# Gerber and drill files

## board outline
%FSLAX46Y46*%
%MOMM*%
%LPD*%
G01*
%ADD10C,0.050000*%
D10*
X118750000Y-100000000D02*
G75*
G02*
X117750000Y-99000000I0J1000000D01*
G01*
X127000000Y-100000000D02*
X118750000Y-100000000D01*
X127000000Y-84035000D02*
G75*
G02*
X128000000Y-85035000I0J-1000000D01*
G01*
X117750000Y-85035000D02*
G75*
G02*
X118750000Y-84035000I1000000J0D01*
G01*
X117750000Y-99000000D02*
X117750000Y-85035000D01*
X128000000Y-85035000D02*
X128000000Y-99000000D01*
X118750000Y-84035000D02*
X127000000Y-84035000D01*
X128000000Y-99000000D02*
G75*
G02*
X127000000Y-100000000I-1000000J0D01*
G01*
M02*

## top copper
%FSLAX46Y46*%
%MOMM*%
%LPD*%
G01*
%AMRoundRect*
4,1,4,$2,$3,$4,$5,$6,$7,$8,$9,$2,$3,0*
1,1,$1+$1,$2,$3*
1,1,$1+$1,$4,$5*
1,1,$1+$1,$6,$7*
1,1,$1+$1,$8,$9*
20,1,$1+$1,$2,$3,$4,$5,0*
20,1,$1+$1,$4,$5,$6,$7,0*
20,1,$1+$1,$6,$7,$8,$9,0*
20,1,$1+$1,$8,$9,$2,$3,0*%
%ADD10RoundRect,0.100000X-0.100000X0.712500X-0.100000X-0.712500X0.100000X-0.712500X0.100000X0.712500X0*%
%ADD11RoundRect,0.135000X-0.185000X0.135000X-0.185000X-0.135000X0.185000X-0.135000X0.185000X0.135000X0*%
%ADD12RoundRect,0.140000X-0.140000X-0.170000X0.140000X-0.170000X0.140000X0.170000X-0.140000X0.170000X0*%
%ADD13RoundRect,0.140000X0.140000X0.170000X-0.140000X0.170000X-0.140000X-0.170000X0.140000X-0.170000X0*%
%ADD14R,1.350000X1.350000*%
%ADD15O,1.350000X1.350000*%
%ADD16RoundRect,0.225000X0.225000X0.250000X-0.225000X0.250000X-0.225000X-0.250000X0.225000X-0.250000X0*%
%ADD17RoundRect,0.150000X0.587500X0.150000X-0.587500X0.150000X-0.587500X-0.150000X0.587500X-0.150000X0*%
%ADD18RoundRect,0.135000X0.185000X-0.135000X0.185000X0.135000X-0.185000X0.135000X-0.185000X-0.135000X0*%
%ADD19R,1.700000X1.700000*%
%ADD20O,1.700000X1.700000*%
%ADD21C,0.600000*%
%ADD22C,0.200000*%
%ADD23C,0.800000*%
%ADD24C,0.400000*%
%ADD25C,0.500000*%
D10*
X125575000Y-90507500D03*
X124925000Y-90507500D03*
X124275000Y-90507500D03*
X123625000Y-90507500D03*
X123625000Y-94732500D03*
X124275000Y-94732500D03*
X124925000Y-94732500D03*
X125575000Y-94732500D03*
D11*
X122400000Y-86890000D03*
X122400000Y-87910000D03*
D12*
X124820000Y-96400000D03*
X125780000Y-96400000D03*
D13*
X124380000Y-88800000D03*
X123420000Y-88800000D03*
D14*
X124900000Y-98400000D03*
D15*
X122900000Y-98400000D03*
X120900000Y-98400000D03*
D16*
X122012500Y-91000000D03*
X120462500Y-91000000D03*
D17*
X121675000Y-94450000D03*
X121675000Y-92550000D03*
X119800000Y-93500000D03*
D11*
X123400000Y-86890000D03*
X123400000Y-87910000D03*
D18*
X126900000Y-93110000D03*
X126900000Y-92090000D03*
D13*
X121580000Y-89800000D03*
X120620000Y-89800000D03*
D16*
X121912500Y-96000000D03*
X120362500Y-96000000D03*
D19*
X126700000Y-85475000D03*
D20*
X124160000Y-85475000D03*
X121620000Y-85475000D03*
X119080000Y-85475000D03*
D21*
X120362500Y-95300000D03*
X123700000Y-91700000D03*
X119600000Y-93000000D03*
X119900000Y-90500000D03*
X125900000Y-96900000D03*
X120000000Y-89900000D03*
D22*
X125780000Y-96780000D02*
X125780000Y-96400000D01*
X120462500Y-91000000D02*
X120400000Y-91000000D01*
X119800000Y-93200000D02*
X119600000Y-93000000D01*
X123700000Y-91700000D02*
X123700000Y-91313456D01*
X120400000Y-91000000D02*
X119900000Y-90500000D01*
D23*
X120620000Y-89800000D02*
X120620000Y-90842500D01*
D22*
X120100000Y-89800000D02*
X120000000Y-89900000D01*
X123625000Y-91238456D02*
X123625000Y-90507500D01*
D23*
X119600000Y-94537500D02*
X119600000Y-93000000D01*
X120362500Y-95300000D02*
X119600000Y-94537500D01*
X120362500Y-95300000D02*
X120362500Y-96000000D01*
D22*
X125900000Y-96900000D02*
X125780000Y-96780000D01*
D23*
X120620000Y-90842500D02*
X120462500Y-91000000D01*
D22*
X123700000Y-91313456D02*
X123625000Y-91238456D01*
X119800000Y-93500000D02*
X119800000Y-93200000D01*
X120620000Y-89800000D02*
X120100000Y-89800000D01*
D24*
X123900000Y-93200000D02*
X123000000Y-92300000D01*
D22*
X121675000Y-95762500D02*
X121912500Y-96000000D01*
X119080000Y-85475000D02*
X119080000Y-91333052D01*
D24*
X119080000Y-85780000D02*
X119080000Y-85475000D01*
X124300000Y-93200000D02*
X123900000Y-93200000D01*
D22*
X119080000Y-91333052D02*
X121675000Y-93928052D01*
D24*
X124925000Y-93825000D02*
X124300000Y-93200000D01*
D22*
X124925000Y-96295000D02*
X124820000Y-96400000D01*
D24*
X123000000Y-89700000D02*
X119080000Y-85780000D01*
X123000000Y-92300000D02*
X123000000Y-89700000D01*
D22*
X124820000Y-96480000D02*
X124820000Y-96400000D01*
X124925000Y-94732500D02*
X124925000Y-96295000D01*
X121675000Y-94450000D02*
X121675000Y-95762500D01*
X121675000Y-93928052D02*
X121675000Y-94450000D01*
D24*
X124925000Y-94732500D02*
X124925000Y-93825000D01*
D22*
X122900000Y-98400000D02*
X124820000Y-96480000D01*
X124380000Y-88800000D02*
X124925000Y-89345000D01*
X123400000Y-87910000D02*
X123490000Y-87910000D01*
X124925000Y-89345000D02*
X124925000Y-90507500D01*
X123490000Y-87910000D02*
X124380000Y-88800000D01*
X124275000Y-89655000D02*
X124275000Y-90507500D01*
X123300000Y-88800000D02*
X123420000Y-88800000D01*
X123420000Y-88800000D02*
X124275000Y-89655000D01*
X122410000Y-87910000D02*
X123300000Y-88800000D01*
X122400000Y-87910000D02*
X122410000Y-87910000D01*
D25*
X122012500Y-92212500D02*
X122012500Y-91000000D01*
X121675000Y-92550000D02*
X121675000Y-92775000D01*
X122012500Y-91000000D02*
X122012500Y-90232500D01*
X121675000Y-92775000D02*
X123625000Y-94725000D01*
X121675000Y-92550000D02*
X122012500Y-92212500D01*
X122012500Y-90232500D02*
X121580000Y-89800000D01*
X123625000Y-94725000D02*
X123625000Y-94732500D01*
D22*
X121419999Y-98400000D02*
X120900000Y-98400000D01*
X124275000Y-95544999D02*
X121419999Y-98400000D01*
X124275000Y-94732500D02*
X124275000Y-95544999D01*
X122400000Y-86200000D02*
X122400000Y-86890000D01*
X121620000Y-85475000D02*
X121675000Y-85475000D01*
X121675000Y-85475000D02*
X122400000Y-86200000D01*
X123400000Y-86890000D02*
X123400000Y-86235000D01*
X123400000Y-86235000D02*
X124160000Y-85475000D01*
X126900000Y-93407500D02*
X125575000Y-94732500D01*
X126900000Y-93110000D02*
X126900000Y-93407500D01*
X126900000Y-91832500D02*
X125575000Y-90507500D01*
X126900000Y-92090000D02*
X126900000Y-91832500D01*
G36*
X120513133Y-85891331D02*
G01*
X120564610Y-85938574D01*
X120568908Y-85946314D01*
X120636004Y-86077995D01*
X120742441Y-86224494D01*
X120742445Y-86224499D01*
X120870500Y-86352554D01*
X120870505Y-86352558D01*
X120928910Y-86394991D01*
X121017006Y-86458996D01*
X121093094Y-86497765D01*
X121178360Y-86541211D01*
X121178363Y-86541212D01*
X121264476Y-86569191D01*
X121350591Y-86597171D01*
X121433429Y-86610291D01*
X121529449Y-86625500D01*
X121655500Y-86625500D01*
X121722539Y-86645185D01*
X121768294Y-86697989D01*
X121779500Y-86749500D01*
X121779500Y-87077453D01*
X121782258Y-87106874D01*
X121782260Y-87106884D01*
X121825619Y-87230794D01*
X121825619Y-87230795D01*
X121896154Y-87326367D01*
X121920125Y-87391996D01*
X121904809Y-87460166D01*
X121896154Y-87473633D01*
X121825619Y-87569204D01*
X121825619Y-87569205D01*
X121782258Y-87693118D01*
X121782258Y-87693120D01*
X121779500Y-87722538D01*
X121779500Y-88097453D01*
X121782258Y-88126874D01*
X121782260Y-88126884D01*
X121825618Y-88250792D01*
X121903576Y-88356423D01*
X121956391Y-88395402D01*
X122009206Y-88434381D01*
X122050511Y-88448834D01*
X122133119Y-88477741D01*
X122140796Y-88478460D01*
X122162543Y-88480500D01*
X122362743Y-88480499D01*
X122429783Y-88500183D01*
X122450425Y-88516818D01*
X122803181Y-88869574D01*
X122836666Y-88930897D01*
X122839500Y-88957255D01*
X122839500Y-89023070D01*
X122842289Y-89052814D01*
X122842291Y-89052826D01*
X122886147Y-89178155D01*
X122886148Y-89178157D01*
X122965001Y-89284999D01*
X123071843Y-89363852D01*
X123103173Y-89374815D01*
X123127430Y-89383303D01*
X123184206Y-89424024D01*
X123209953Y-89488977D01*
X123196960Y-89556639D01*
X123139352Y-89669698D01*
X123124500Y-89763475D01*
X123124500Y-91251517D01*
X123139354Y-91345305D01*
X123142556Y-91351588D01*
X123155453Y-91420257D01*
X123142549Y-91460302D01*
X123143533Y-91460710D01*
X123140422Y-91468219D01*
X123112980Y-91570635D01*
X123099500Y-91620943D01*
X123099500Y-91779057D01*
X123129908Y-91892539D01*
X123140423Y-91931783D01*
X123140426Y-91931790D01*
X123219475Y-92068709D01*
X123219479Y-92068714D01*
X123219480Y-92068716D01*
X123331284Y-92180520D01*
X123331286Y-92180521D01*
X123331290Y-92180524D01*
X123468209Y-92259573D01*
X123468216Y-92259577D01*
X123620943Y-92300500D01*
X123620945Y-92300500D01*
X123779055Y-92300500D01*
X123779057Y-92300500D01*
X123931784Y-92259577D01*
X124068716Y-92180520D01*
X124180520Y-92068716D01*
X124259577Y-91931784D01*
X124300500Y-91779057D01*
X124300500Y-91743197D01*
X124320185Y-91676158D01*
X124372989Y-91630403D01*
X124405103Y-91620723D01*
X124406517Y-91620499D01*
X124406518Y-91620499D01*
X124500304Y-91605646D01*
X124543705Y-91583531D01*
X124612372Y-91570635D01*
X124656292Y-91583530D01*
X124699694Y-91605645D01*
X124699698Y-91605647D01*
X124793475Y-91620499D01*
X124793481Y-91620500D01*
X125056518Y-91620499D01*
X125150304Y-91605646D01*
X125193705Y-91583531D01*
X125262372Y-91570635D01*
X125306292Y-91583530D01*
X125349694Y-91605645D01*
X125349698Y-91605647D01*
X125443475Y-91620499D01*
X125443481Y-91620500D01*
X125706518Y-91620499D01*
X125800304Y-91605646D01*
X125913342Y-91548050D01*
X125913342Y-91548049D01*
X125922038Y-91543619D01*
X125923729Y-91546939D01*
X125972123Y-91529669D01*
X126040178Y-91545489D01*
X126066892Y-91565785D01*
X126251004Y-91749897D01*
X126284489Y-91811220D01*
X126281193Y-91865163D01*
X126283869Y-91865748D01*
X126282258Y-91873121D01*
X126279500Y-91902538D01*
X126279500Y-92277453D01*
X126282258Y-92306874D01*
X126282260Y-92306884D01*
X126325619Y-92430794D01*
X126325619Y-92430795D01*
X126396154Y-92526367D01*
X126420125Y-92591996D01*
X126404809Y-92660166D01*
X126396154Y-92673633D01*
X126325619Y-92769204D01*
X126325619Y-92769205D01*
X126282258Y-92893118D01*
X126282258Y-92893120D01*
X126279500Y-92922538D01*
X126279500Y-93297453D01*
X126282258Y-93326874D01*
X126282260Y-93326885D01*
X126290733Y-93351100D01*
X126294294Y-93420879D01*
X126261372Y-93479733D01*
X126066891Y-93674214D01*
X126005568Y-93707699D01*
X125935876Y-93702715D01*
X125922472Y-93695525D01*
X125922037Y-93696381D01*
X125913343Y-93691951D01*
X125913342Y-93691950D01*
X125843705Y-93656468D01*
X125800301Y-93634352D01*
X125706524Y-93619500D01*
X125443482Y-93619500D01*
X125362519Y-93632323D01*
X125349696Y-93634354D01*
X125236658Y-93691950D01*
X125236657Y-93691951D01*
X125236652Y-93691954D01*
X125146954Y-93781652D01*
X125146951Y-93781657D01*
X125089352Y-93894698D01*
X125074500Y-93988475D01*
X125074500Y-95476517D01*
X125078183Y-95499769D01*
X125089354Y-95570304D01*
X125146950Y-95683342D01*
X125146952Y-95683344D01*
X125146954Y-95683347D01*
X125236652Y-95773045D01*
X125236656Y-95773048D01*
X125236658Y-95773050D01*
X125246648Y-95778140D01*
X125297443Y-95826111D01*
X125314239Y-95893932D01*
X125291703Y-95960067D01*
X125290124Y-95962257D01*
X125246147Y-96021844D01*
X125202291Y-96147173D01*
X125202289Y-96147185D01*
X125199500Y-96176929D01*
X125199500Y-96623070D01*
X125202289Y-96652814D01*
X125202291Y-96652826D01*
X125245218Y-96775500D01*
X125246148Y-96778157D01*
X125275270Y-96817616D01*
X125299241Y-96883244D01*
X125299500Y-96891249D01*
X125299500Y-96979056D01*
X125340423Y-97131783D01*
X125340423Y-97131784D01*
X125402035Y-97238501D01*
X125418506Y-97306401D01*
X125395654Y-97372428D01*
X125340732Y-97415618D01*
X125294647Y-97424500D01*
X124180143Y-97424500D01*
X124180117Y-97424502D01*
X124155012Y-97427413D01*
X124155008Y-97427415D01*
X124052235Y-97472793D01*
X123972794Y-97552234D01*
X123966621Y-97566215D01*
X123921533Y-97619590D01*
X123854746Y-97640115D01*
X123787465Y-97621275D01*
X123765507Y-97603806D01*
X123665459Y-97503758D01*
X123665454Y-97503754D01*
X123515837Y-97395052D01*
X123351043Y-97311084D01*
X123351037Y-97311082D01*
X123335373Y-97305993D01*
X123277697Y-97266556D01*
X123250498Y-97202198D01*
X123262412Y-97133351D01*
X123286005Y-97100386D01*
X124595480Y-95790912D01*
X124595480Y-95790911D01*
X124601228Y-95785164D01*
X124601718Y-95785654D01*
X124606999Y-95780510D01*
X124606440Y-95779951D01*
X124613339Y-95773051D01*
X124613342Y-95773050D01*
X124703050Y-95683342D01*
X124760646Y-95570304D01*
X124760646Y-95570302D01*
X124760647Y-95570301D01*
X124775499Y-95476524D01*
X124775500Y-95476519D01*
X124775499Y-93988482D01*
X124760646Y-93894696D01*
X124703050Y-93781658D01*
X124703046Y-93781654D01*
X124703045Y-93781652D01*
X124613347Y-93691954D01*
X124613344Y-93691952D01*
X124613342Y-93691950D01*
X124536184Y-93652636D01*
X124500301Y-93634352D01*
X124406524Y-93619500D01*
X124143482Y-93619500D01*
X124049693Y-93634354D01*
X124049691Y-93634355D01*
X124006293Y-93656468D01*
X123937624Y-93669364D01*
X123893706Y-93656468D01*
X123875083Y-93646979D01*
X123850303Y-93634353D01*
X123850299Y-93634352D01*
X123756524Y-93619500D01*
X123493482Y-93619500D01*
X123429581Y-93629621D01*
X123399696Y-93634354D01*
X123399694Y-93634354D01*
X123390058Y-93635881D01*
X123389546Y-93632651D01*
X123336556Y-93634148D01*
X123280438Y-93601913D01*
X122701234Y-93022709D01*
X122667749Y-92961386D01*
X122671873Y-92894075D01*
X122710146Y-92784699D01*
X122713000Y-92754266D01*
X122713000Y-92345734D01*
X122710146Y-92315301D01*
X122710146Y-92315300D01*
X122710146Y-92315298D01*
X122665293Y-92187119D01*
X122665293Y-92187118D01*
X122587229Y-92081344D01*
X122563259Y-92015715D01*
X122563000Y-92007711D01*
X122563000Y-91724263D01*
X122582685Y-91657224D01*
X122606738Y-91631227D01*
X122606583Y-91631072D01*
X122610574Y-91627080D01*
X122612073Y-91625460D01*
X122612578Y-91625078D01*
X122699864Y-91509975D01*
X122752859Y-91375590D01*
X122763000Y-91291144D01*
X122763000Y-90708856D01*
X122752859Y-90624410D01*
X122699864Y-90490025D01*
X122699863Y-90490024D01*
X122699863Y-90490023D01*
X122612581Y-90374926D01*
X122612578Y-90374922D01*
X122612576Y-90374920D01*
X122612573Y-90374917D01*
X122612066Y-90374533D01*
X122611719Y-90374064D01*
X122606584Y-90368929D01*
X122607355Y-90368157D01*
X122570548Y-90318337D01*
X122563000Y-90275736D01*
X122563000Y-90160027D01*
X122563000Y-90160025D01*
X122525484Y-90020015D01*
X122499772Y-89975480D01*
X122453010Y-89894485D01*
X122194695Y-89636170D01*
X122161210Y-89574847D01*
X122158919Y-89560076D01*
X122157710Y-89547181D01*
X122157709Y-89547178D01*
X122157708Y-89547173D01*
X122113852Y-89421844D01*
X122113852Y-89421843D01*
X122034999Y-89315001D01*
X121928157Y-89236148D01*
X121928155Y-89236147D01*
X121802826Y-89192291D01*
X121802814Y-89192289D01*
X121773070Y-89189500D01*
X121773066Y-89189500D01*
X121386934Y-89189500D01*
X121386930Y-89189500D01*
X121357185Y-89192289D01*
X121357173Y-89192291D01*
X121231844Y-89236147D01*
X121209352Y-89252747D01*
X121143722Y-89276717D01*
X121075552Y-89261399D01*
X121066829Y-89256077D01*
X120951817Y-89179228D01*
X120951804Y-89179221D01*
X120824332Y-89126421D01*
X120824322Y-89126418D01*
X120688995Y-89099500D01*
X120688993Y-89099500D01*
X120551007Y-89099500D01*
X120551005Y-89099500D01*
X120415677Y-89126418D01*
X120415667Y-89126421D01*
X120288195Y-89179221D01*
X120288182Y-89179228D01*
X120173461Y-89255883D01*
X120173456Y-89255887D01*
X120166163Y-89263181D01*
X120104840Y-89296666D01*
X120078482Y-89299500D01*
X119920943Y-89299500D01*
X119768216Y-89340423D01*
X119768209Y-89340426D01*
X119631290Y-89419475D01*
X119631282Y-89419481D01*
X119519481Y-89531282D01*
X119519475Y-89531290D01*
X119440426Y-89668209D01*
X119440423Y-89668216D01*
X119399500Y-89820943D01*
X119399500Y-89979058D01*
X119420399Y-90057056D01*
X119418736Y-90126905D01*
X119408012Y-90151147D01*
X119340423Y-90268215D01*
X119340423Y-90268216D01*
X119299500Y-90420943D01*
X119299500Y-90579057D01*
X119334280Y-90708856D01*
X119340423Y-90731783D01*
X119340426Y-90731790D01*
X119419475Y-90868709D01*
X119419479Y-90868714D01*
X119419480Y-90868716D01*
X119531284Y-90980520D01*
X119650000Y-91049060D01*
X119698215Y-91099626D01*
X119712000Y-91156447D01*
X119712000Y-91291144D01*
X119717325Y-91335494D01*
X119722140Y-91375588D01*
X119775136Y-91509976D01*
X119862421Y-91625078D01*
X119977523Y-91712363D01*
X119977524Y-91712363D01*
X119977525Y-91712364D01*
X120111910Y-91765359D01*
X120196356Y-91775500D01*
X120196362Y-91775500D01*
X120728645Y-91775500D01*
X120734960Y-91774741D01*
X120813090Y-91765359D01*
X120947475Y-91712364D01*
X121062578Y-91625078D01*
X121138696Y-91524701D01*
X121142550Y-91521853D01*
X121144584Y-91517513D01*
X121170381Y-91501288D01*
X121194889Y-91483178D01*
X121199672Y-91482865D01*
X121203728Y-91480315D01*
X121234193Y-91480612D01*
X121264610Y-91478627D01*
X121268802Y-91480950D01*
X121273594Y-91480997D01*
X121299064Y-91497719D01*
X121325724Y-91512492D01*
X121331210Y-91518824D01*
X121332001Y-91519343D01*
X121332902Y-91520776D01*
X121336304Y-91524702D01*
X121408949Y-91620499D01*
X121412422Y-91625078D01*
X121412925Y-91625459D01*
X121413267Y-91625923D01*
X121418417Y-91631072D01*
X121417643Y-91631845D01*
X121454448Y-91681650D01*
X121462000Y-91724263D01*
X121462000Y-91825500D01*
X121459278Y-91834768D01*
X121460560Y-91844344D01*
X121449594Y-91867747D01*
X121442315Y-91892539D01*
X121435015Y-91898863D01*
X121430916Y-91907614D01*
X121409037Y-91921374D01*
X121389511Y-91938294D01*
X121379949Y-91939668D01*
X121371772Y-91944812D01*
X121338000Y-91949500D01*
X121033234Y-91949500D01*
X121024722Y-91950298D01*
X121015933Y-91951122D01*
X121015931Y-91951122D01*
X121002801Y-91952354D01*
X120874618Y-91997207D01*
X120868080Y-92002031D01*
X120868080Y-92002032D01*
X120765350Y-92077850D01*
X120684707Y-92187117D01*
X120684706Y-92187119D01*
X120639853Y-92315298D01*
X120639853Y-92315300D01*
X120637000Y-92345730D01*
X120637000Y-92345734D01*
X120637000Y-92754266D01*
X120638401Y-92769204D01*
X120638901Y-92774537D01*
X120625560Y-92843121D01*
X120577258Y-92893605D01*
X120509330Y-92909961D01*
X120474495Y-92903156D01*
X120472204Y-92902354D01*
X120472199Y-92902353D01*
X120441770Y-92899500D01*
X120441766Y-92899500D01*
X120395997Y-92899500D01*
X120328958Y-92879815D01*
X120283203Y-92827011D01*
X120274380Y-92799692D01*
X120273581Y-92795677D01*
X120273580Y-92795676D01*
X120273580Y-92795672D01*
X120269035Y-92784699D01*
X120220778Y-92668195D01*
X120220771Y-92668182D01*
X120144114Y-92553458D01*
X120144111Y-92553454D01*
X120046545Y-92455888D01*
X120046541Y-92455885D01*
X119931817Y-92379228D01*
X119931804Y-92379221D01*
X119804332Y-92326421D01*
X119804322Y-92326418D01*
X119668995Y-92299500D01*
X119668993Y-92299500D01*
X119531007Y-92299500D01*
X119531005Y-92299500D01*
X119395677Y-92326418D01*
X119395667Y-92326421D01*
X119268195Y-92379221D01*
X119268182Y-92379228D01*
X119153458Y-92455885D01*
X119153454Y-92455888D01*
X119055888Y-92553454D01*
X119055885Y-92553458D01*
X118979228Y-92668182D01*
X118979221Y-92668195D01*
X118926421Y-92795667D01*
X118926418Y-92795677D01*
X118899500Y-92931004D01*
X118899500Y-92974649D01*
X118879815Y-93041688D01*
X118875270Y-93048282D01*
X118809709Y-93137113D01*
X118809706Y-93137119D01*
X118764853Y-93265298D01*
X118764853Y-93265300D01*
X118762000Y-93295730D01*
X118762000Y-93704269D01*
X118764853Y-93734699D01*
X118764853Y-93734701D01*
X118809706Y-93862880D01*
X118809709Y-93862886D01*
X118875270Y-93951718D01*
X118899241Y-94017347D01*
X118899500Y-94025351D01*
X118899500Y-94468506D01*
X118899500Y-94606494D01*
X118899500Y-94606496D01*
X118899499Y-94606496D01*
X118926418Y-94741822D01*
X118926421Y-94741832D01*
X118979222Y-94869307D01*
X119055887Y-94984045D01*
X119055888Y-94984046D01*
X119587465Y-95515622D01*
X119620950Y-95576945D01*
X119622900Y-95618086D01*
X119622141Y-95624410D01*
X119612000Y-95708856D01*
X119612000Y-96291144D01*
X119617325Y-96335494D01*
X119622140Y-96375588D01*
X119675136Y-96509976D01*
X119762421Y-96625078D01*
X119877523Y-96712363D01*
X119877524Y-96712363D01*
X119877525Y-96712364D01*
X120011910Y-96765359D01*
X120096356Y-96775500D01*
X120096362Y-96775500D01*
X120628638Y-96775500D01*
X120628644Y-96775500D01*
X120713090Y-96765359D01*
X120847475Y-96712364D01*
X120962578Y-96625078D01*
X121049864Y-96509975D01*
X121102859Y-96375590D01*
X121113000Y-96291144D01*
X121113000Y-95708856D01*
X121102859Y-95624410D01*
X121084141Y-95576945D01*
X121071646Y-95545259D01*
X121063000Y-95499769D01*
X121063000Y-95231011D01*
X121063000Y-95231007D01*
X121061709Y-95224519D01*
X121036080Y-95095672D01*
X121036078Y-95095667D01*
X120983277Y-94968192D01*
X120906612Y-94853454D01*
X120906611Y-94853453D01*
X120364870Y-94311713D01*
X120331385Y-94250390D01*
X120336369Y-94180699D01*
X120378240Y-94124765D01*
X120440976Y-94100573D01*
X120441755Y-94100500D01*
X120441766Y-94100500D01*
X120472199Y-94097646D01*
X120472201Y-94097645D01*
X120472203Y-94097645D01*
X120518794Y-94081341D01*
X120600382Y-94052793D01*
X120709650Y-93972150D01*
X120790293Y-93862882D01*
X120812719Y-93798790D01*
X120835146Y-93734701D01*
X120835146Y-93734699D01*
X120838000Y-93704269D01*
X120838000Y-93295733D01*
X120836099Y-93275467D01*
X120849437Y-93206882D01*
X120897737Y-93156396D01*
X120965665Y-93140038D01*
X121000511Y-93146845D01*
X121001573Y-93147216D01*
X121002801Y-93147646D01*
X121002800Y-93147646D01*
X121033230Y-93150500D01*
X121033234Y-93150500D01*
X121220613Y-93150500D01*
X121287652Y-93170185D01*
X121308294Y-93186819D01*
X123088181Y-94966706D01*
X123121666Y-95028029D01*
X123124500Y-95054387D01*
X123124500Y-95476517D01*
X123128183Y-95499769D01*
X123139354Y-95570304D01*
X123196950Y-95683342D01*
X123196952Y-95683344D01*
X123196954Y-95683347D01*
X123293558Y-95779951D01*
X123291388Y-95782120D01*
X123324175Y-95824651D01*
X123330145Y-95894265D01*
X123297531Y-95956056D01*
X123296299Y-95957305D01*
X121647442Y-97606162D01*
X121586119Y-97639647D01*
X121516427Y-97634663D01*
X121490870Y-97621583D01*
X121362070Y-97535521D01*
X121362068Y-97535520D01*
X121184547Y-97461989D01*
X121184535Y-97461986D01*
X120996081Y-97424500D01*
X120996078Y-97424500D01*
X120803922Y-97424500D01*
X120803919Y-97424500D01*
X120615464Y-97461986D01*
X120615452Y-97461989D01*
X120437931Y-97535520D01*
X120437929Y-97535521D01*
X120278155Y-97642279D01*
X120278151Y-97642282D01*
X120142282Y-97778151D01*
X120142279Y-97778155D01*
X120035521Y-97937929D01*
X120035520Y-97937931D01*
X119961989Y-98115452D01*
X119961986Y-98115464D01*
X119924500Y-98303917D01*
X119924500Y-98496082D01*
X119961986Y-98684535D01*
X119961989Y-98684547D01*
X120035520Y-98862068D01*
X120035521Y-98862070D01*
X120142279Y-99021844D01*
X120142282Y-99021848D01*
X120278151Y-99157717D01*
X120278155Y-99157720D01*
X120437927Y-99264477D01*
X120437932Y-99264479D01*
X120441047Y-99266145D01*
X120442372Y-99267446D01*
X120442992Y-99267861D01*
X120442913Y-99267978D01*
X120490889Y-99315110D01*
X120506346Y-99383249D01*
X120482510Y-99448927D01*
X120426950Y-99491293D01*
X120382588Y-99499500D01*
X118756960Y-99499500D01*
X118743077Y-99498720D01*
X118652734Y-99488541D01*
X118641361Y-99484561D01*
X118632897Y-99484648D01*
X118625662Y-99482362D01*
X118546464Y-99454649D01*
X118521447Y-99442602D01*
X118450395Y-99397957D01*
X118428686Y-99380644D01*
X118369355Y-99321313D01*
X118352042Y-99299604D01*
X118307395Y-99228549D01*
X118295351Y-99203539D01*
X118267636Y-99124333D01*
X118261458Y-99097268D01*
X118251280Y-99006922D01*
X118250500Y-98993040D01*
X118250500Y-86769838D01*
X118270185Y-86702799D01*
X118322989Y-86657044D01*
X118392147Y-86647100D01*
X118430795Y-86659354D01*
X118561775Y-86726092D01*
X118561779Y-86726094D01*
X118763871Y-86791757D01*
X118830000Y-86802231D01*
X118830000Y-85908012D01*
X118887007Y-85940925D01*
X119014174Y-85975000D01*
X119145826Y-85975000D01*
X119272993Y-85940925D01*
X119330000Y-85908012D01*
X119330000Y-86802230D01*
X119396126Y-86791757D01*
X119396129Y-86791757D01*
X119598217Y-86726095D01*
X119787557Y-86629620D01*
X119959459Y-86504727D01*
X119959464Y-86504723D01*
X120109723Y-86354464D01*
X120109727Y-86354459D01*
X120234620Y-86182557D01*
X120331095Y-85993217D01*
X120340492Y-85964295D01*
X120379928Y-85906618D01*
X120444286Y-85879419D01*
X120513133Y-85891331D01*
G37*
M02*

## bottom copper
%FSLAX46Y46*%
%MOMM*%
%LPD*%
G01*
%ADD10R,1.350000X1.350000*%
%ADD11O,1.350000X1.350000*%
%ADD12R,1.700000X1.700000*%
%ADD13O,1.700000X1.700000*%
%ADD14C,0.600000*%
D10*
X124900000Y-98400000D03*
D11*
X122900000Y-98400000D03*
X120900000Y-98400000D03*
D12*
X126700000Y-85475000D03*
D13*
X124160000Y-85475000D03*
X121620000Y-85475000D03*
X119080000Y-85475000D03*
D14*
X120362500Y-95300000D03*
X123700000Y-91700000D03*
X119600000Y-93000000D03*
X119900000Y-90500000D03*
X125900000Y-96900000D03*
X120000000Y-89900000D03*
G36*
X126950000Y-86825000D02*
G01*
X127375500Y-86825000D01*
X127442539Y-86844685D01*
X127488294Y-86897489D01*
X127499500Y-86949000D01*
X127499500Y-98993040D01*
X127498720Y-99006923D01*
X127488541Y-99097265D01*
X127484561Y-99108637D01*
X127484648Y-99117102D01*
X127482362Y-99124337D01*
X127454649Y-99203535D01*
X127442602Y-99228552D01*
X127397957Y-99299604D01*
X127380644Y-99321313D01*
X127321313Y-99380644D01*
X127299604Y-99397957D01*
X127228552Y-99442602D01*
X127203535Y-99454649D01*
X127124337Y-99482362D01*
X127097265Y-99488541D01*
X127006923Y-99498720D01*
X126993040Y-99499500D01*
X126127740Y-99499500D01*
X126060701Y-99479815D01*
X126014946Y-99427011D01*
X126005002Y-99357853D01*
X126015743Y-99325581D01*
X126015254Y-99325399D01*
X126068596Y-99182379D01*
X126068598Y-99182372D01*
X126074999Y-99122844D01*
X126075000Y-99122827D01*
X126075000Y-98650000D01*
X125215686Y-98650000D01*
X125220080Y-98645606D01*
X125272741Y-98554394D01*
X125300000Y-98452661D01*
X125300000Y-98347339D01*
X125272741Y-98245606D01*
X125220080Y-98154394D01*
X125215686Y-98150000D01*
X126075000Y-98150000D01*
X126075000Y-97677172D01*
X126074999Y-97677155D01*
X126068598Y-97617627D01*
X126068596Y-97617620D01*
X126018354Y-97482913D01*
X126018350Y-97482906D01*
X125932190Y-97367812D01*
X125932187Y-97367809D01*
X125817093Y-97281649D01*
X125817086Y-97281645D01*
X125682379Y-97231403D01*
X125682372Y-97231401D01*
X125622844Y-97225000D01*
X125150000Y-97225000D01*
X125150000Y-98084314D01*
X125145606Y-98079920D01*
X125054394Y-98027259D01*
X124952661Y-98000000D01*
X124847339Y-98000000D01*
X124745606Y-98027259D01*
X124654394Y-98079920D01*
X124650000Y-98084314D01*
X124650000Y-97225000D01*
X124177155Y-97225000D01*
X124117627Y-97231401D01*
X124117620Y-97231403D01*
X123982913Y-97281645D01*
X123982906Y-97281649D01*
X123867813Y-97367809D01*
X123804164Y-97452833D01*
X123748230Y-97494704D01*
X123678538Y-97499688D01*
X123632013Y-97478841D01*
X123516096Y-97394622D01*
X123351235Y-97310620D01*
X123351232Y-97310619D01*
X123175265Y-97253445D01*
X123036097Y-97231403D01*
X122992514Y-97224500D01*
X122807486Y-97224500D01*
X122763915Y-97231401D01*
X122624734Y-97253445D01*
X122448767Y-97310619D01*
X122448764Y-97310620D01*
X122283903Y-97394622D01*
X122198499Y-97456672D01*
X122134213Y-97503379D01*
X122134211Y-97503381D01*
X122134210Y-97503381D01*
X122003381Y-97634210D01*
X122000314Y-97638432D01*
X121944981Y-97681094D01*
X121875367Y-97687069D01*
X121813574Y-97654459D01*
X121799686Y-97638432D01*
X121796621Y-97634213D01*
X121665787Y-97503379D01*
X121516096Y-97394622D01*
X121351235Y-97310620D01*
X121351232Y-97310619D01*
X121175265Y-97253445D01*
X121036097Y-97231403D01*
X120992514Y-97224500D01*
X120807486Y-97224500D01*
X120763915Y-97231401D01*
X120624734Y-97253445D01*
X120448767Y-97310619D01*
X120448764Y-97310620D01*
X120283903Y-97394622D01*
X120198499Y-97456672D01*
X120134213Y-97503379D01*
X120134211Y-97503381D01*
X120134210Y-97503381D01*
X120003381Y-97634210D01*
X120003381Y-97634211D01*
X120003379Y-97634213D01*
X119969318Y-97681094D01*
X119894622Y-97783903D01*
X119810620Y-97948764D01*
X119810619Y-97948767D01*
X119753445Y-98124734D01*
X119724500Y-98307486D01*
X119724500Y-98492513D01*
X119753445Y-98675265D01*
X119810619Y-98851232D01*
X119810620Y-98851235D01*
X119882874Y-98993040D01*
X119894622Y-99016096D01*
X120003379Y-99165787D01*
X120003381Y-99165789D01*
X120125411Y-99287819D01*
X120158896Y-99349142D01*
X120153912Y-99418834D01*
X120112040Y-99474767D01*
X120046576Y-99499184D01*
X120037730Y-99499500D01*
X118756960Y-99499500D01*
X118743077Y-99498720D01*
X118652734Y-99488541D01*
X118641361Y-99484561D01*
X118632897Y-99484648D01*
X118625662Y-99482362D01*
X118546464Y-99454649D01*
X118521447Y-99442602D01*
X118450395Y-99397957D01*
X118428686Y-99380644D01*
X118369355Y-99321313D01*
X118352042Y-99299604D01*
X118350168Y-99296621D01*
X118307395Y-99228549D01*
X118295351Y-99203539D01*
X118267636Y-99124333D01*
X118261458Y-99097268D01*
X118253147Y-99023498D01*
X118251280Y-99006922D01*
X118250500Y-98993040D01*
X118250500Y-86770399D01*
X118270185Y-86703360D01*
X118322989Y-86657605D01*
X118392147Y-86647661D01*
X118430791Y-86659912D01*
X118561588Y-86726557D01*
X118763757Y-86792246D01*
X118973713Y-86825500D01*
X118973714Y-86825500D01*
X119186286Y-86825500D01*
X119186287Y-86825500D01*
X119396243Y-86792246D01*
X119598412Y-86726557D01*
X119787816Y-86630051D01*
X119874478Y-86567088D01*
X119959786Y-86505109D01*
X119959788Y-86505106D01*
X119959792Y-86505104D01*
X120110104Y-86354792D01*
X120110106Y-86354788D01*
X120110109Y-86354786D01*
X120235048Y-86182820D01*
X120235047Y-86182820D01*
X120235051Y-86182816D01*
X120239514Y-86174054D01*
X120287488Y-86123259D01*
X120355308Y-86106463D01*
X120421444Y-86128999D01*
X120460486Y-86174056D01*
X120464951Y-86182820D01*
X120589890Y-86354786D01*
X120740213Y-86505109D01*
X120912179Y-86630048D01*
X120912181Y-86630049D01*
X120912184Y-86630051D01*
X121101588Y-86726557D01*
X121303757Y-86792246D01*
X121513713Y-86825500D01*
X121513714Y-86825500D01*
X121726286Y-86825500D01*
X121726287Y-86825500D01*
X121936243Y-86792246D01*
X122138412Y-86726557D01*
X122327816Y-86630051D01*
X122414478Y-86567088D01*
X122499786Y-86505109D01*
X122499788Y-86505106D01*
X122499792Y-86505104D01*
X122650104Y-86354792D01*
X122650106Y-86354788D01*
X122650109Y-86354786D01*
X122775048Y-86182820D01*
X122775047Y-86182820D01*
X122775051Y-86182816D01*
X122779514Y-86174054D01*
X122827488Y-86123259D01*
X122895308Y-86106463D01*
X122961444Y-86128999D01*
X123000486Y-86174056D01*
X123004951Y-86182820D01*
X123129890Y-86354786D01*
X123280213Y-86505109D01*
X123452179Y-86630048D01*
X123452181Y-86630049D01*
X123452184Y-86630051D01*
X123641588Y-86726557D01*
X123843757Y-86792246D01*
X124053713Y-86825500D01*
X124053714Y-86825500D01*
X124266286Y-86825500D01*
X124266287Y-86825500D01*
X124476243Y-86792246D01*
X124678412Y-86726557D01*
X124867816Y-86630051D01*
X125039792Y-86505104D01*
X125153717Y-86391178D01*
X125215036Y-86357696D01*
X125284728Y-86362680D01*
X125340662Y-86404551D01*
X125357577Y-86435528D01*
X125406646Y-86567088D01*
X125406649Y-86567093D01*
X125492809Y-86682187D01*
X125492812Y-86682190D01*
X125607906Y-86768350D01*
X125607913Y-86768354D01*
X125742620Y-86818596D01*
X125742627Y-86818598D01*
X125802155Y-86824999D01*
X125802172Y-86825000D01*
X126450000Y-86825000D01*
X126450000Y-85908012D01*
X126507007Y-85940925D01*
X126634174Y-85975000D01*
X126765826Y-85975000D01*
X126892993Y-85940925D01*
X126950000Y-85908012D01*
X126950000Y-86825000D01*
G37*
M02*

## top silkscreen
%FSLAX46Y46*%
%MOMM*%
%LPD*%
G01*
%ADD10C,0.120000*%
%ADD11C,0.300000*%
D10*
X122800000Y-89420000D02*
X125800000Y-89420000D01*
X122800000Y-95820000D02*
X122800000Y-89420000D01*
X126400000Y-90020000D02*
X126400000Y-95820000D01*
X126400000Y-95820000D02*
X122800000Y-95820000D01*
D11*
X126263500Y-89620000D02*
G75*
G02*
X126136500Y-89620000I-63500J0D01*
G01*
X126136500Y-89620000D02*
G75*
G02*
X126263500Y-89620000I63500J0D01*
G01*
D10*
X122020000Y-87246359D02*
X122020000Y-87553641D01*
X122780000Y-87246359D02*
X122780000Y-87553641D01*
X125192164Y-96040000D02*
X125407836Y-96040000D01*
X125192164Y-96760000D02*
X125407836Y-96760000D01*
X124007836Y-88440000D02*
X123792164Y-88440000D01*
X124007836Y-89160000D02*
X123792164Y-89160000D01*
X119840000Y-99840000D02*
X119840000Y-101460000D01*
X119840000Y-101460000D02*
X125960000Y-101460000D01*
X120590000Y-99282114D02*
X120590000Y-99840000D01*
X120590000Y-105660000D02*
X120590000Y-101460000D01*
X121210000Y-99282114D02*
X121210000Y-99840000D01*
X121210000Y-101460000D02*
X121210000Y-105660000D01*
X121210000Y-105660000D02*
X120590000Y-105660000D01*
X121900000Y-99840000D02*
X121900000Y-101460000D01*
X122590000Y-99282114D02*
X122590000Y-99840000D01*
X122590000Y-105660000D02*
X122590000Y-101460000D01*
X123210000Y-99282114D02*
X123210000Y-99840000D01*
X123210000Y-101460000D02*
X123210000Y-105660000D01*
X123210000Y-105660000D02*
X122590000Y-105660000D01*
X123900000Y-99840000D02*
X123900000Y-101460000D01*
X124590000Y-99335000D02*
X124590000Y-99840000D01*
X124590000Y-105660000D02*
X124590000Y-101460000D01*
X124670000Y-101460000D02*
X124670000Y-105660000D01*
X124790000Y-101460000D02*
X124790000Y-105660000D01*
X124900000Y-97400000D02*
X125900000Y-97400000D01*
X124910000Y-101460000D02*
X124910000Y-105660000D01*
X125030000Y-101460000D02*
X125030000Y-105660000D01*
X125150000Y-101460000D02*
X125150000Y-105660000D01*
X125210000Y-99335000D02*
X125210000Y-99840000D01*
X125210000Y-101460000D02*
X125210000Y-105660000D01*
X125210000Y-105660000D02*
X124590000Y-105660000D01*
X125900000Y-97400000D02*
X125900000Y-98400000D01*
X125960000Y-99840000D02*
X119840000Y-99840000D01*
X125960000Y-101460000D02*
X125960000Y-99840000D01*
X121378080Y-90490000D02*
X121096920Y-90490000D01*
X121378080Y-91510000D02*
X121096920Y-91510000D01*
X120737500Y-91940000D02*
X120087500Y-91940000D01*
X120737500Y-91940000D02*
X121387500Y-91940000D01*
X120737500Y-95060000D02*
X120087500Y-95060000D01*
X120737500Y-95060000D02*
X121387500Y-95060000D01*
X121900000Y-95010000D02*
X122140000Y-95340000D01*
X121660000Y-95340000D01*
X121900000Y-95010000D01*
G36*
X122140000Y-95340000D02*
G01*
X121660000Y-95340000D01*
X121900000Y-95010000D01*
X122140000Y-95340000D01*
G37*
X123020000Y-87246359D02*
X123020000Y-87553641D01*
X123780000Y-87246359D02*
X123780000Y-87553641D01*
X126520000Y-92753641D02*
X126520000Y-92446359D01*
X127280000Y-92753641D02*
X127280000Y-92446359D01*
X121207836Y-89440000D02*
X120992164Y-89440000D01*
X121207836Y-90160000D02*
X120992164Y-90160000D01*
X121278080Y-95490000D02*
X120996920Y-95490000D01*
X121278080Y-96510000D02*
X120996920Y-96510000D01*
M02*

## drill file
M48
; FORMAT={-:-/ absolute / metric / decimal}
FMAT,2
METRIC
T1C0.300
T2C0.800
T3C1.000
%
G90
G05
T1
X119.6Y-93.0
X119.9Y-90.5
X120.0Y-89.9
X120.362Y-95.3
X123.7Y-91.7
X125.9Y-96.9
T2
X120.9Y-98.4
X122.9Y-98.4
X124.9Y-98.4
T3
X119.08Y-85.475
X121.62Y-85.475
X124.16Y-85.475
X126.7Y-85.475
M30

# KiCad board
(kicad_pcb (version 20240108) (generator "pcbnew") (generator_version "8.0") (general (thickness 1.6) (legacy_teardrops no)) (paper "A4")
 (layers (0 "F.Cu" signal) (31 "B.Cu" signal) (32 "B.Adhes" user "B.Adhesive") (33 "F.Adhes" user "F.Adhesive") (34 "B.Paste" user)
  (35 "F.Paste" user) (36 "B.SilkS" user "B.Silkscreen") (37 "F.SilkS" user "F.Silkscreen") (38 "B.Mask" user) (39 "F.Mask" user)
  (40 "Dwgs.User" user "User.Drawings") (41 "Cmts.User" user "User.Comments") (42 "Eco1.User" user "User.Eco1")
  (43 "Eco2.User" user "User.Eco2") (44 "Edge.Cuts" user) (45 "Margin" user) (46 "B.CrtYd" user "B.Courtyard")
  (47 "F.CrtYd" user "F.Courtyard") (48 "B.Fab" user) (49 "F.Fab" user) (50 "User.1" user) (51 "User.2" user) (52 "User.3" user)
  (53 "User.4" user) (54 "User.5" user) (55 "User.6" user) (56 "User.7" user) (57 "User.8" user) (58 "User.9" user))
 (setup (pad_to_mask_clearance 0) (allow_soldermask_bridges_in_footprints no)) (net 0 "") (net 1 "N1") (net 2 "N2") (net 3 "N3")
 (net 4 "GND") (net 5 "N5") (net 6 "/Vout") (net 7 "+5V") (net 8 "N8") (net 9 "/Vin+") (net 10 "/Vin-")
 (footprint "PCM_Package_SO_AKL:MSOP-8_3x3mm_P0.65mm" (layer "F.Cu") (at 124.6 92.62 -90)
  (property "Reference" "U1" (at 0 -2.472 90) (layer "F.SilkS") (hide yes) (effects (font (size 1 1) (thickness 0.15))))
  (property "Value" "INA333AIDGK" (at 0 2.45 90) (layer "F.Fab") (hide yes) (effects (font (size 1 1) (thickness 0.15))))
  (fp_line (start -3.2 1.8) (end -3.2 -1.2) (stroke (width 0.12) (type solid)) (layer "F.SilkS"))
  (fp_line (start 3.2 1.8) (end -3.2 1.8) (stroke (width 0.12) (type solid)) (layer "F.SilkS"))
  (fp_line (start -2.6 -1.8) (end 3.2 -1.8) (stroke (width 0.12) (type solid)) (layer "F.SilkS"))
  (fp_line (start 3.2 -1.8) (end 3.2 1.8) (stroke (width 0.12) (type solid)) (layer "F.SilkS"))
  (fp_circle (center -3 -1.6) (end -2.9365 -1.6) (stroke (width 0.3) (type solid)) (fill none) (layer "F.SilkS"))
  (pad "1" smd roundrect (at -2.1125 -0.975 270) (size 1.625 0.4) (layers "F.Cu" "F.Paste" "F.Mask") (roundrect_rratio 0.25) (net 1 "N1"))
  (pad "2" smd roundrect (at -2.1125 -0.325 270) (size 1.625 0.4) (layers "F.Cu" "F.Paste" "F.Mask") (roundrect_rratio 0.25) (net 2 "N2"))
  (pad "3" smd roundrect (at -2.1125 0.325 270) (size 1.625 0.4) (layers "F.Cu" "F.Paste" "F.Mask") (roundrect_rratio 0.25) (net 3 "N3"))
  (pad "4" smd roundrect (at -2.1125 0.975 270) (size 1.625 0.4) (layers "F.Cu" "F.Paste" "F.Mask") (roundrect_rratio 0.25) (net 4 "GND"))
  (pad "5" smd roundrect (at 2.1125 0.975 270) (size 1.625 0.4) (layers "F.Cu" "F.Paste" "F.Mask") (roundrect_rratio 0.25) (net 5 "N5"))
  (pad "6" smd roundrect (at 2.1125 0.325 270) (size 1.625 0.4) (layers "F.Cu" "F.Paste" "F.Mask") (roundrect_rratio 0.25) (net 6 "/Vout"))
  (pad "7" smd roundrect (at 2.1125 -0.325 270) (size 1.625 0.4) (layers "F.Cu" "F.Paste" "F.Mask") (roundrect_rratio 0.25) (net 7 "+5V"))
  (pad "8" smd roundrect (at 2.1125 -0.975 270) (size 1.625 0.4) (layers "F.Cu" "F.Paste" "F.Mask") (roundrect_rratio 0.25) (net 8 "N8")))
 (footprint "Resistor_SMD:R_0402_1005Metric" (layer "F.Cu") (at 122.4 87.4 -90)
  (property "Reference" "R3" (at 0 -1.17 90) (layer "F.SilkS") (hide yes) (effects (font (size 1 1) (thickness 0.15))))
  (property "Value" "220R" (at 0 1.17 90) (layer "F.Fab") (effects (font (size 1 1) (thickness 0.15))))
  (fp_line (start -0.153641 0.38) (end 0.153641 0.38) (stroke (width 0.12) (type solid)) (layer "F.SilkS"))
  (fp_line (start -0.153641 -0.38) (end 0.153641 -0.38) (stroke (width 0.12) (type solid)) (layer "F.SilkS"))
  (pad "1" smd roundrect (at -0.51 0 270) (size 0.54 0.64) (layers "F.Cu" "F.Paste" "F.Mask") (roundrect_rratio 0.25) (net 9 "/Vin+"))
  (pad "2" smd roundrect (at 0.51 0 270) (size 0.54 0.64) (layers "F.Cu" "F.Paste" "F.Mask") (roundrect_rratio 0.25) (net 3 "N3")))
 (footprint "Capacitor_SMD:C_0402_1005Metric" (layer "F.Cu") (at 125.3 96.4)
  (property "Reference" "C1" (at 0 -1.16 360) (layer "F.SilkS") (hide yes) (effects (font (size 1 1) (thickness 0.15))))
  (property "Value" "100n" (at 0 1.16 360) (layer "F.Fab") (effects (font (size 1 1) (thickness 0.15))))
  (fp_line (start -0.107836 -0.36) (end 0.107836 -0.36) (stroke (width 0.12) (type solid)) (layer "F.SilkS"))
  (fp_line (start -0.107836 0.36) (end 0.107836 0.36) (stroke (width 0.12) (type solid)) (layer "F.SilkS"))
  (pad "1" smd roundrect (at -0.48 0) (size 0.56 0.62) (layers "F.Cu" "F.Paste" "F.Mask") (roundrect_rratio 0.25) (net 7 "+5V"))
  (pad "2" smd roundrect (at 0.48 0) (size 0.56 0.62) (layers "F.Cu" "F.Paste" "F.Mask") (roundrect_rratio 0.25) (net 4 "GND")))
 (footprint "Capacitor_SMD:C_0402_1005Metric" (layer "F.Cu") (at 123.9 88.8 180)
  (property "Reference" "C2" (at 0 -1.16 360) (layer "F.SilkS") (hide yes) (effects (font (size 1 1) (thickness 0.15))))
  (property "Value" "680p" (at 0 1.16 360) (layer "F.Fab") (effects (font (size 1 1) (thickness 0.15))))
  (fp_line (start -0.107836 0.36) (end 0.107836 0.36) (stroke (width 0.12) (type solid)) (layer "F.SilkS"))
  (fp_line (start -0.107836 -0.36) (end 0.107836 -0.36) (stroke (width 0.12) (type solid)) (layer "F.SilkS"))
  (pad "1" smd roundrect (at -0.48 0 180) (size 0.56 0.62) (layers "F.Cu" "F.Paste" "F.Mask") (roundrect_rratio 0.25) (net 2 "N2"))
  (pad "2" smd roundrect (at 0.48 0 180) (size 0.56 0.62) (layers "F.Cu" "F.Paste" "F.Mask") (roundrect_rratio 0.25) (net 3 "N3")))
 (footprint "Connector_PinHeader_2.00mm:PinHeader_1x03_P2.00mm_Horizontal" (layer "F.Cu") (at 124.9 98.4 -90)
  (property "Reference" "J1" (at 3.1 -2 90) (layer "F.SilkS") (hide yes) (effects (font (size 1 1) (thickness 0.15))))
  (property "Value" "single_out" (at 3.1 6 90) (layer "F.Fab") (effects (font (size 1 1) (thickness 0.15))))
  (fp_line (start 1.44 5.06) (end 3.06 5.06) (stroke (width 0.12) (type solid)) (layer "F.SilkS"))
  (fp_line (start 3.06 5.06) (end 3.06 -1.06) (stroke (width 0.12) (type solid)) (layer "F.SilkS"))
  (fp_line (start 0.882114 4.31) (end 1.44 4.31) (stroke (width 0.12) (type solid)) (layer "F.SilkS"))
  (fp_line (start 7.26 4.31) (end 3.06 4.31) (stroke (width 0.12) (type solid)) (layer "F.SilkS"))
  (fp_line (start 0.882114 3.69) (end 1.44 3.69) (stroke (width 0.12) (type solid)) (layer "F.SilkS"))
  (fp_line (start 3.06 3.69) (end 7.26 3.69) (stroke (width 0.12) (type solid)) (layer "F.SilkS"))
  (fp_line (start 7.26 3.69) (end 7.26 4.31) (stroke (width 0.12) (type solid)) (layer "F.SilkS"))
  (fp_line (start 1.44 3) (end 3.06 3) (stroke (width 0.12) (type solid)) (layer "F.SilkS"))
  (fp_line (start 0.882114 2.31) (end 1.44 2.31) (stroke (width 0.12) (type solid)) (layer "F.SilkS"))
  (fp_line (start 7.26 2.31) (end 3.06 2.31) (stroke (width 0.12) (type solid)) (layer "F.SilkS"))
  (fp_line (start 0.882114 1.69) (end 1.44 1.69) (stroke (width 0.12) (type solid)) (layer "F.SilkS"))
  (fp_line (start 3.06 1.69) (end 7.26 1.69) (stroke (width 0.12) (type solid)) (layer "F.SilkS"))
  (fp_line (start 7.26 1.69) (end 7.26 2.31) (stroke (width 0.12) (type solid)) (layer "F.SilkS"))
  (fp_line (start 1.44 1) (end 3.06 1) (stroke (width 0.12) (type solid)) (layer "F.SilkS"))
  (fp_line (start 0.935 0.31) (end 1.44 0.31) (stroke (width 0.12) (type solid)) (layer "F.SilkS"))
  (fp_line (start 7.26 0.31) (end 3.06 0.31) (stroke (width 0.12) (type solid)) (layer "F.SilkS"))
  (fp_line (start 3.06 0.23) (end 7.26 0.23) (stroke (width 0.12) (type solid)) (layer "F.SilkS"))
  (fp_line (start 3.06 0.11) (end 7.26 0.11) (stroke (width 0.12) (type solid)) (layer "F.SilkS"))
  (fp_line (start -1 0) (end -1 -1) (stroke (width 0.12) (type solid)) (layer "F.SilkS"))
  (fp_line (start 3.06 -0.01) (end 7.26 -0.01) (stroke (width 0.12) (type solid)) (layer "F.SilkS"))
  (fp_line (start 3.06 -0.13) (end 7.26 -0.13) (stroke (width 0.12) (type solid)) (layer "F.SilkS"))
  (fp_line (start 3.06 -0.25) (end 7.26 -0.25) (stroke (width 0.12) (type solid)) (layer "F.SilkS"))
  (fp_line (start 0.935 -0.31) (end 1.44 -0.31) (stroke (width 0.12) (type solid)) (layer "F.SilkS"))
  (fp_line (start 3.06 -0.31) (end 7.26 -0.31) (stroke (width 0.12) (type solid)) (layer "F.SilkS"))
  (fp_line (start 7.26 -0.31) (end 7.26 0.31) (stroke (width 0.12) (type solid)) (layer "F.SilkS"))
  (fp_line (start -1 -1) (end 0 -1) (stroke (width 0.12) (type solid)) (layer "F.SilkS"))
  (fp_line (start 1.44 -1.06) (end 1.44 5.06) (stroke (width 0.12) (type solid)) (layer "F.SilkS"))
  (fp_line (start 3.06 -1.06) (end 1.44 -1.06) (stroke (width 0.12) (type solid)) (layer "F.SilkS"))
  (pad "1" thru_hole rect (at 0 0 270) (size 1.35 1.35) (drill 0.8) (layers "*.Cu" "*.Mask") (remove_unused_layers no) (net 4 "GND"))
  (pad "2" thru_hole oval (at 0 2 270) (size 1.35 1.35) (drill 0.8) (layers "*.Cu" "*.Mask") (remove_unused_layers no) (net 7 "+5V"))
  (pad "3" thru_hole oval (at 0 4 270) (size 1.35 1.35) (drill 0.8) (layers "*.Cu" "*.Mask") (remove_unused_layers no) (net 6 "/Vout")))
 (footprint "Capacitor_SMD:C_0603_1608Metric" (layer "F.Cu") (at 121.2375 91 180)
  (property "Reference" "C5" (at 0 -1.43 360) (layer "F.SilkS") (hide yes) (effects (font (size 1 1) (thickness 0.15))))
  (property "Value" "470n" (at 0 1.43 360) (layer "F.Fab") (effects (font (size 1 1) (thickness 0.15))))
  (fp_line (start -0.14058 0.51) (end 0.14058 0.51) (stroke (width 0.12) (type solid)) (layer "F.SilkS"))
  (fp_line (start -0.14058 -0.51) (end 0.14058 -0.51) (stroke (width 0.12) (type solid)) (layer "F.SilkS"))
  (pad "1" smd roundrect (at -0.775 0 180) (size 0.9 0.95) (layers "F.Cu" "F.Paste" "F.Mask") (roundrect_rratio 0.25) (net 5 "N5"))
  (pad "2" smd roundrect (at 0.775 0 180) (size 0.9 0.95) (layers "F.Cu" "F.Paste" "F.Mask") (roundrect_rratio 0.25) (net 4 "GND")))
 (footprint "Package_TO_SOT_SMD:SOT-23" (layer "F.Cu") (at 120.7375 93.5 180)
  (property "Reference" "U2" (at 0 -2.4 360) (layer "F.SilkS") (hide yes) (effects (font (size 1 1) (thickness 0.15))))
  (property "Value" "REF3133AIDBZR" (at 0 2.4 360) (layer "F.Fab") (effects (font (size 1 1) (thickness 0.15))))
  (fp_line (start 0 1.56) (end 0.65 1.56) (stroke (width 0.12) (type solid)) (layer "F.SilkS"))
  (fp_line (start 0 1.56) (end -0.65 1.56) (stroke (width 0.12) (type solid)) (layer "F.SilkS"))
  (fp_line (start 0 -1.56) (end 0.65 -1.56) (stroke (width 0.12) (type solid)) (layer "F.SilkS"))
  (fp_line (start 0 -1.56) (end -0.65 -1.56) (stroke (width 0.12) (type solid)) (layer "F.SilkS"))
  (fp_poly
   (pts (xy -1.1625 -1.51) (xy -1.4025 -1.84) (xy -0.9225 -1.84) (xy -1.1625 -1.51)) (stroke (width 0.12) (type solid)) (fill solid)
   (layer "F.SilkS"))
  (pad "1" smd roundrect (at -0.9375 -0.95 180) (size 1.475 0.6) (layers "F.Cu" "F.Paste" "F.Mask") (roundrect_rratio 0.25) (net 7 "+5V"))
  (pad "2" smd roundrect (at -0.9375 0.95 180) (size 1.475 0.6) (layers "F.Cu" "F.Paste" "F.Mask") (roundrect_rratio 0.25) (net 5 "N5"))
  (pad "3" smd roundrect (at 0.9375 0 180) (size 1.475 0.6) (layers "F.Cu" "F.Paste" "F.Mask") (roundrect_rratio 0.25) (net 4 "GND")))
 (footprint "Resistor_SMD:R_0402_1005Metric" (layer "F.Cu") (at 123.4 87.4 -90)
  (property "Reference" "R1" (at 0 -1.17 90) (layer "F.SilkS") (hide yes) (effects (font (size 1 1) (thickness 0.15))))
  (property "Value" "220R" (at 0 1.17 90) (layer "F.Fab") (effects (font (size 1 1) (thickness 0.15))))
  (fp_line (start -0.153641 0.38) (end 0.153641 0.38) (stroke (width 0.12) (type solid)) (layer "F.SilkS"))
  (fp_line (start -0.153641 -0.38) (end 0.153641 -0.38) (stroke (width 0.12) (type solid)) (layer "F.SilkS"))
  (pad "1" smd roundrect (at -0.51 0 270) (size 0.54 0.64) (layers "F.Cu" "F.Paste" "F.Mask") (roundrect_rratio 0.25) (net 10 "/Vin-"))
  (pad "2" smd roundrect (at 0.51 0 270) (size 0.54 0.64) (layers "F.Cu" "F.Paste" "F.Mask") (roundrect_rratio 0.25) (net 2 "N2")))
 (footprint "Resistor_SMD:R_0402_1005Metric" (layer "F.Cu") (at 126.9 92.6 90)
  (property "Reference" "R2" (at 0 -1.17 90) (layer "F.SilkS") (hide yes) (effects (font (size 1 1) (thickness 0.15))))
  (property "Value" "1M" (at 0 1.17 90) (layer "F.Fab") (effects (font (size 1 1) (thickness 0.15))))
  (fp_line (start -0.153641 -0.38) (end 0.153641 -0.38) (stroke (width 0.12) (type solid)) (layer "F.SilkS"))
  (fp_line (start -0.153641 0.38) (end 0.153641 0.38) (stroke (width 0.12) (type solid)) (layer "F.SilkS"))
  (pad "1" smd roundrect (at -0.51 0 90) (size 0.54 0.64) (layers "F.Cu" "F.Paste" "F.Mask") (roundrect_rratio 0.25) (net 8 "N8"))
  (pad "2" smd roundrect (at 0.51 0 90) (size 0.54 0.64) (layers "F.Cu" "F.Paste" "F.Mask") (roundrect_rratio 0.25) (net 1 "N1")))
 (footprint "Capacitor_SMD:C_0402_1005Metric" (layer "F.Cu") (at 121.1 89.8 180)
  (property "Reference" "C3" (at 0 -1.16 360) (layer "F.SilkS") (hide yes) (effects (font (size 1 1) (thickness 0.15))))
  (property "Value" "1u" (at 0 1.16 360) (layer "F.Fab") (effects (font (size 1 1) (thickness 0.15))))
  (fp_line (start -0.107836 0.36) (end 0.107836 0.36) (stroke (width 0.12) (type solid)) (layer "F.SilkS"))
  (fp_line (start -0.107836 -0.36) (end 0.107836 -0.36) (stroke (width 0.12) (type solid)) (layer "F.SilkS"))
  (pad "1" smd roundrect (at -0.48 0 180) (size 0.56 0.62) (layers "F.Cu" "F.Paste" "F.Mask") (roundrect_rratio 0.25) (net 5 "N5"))
  (pad "2" smd roundrect (at 0.48 0 180) (size 0.56 0.62) (layers "F.Cu" "F.Paste" "F.Mask") (roundrect_rratio 0.25) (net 4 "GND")))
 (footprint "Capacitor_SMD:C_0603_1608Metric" (layer "F.Cu") (at 121.1375 96 180)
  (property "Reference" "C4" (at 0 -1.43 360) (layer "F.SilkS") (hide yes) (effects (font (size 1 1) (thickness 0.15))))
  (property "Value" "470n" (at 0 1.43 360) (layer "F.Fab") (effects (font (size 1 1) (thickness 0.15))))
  (fp_line (start -0.14058 0.51) (end 0.14058 0.51) (stroke (width 0.12) (type solid)) (layer "F.SilkS"))
  (fp_line (start -0.14058 -0.51) (end 0.14058 -0.51) (stroke (width 0.12) (type solid)) (layer "F.SilkS"))
  (pad "1" smd roundrect (at -0.775 0 180) (size 0.9 0.95) (layers "F.Cu" "F.Paste" "F.Mask") (roundrect_rratio 0.25) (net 7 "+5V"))
  (pad "2" smd roundrect (at 0.775 0 180) (size 0.9 0.95) (layers "F.Cu" "F.Paste" "F.Mask") (roundrect_rratio 0.25) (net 4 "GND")))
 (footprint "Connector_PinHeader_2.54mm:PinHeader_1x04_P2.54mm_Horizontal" (layer "B.Cu") (at 126.7 85.475 90)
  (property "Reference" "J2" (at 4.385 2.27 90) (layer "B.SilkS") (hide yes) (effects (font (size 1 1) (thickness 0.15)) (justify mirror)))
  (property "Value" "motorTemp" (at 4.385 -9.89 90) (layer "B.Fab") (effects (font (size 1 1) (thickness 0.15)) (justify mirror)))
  (pad "1" thru_hole rect (at 0 0 90) (size 1.7 1.7) (drill 1) (layers "*.Cu" "*.Mask") (remove_unused_layers no) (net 4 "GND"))
  (pad "2" thru_hole oval (at 0 -2.54 90) (size 1.7 1.7) (drill 1) (layers "*.Cu" "*.Mask") (remove_unused_layers no) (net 10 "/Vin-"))
  (pad "3" thru_hole oval (at 0 -5.08 90) (size 1.7 1.7) (drill 1) (layers "*.Cu" "*.Mask") (remove_unused_layers no) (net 9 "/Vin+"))
  (pad "4" thru_hole oval (at 0 -7.62 90) (size 1.7 1.7) (drill 1) (layers "*.Cu" "*.Mask") (remove_unused_layers no) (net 7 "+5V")))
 (gr_arc (start 118.75 100) (mid 118.042893 99.707107) (end 117.75 99) (stroke (width 0.05) (type default)) (layer "Edge.Cuts"))
 (gr_line (start 127 100) (end 118.75 100) (stroke (width 0.05) (type default)) (layer "Edge.Cuts"))
 (gr_arc (start 127 84.035) (mid 127.707107 84.327893) (end 128 85.035) (stroke (width 0.05) (type default)) (layer "Edge.Cuts"))
 (gr_arc (start 117.75 85.035) (mid 118.042893 84.327893) (end 118.75 84.035) (stroke (width 0.05) (type default)) (layer "Edge.Cuts"))
 (gr_line (start 117.75 99) (end 117.75 85.035) (stroke (width 0.05) (type default)) (layer "Edge.Cuts"))
 (gr_line (start 128 85.035) (end 128 99) (stroke (width 0.05) (type default)) (layer "Edge.Cuts"))
 (gr_line (start 118.75 84.035) (end 127 84.035) (stroke (width 0.05) (type default)) (layer "Edge.Cuts"))
 (gr_arc (start 128 99) (mid 127.707107 99.707107) (end 127 100) (stroke (width 0.05) (type default)) (layer "Edge.Cuts"))
 (segment (start 125.78 96.78) (end 125.78 96.4) (width 0.2) (layer "F.Cu") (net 4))
 (segment (start 120.4625 91) (end 120.4 91) (width 0.2) (layer "F.Cu") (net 4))
 (segment (start 119.8 93.2) (end 119.6 93) (width 0.2) (layer "F.Cu") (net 4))
 (segment (start 123.7 91.7) (end 123.7 91.313456) (width 0.2) (layer "F.Cu") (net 4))
 (segment (start 120.4 91) (end 119.9 90.5) (width 0.2) (layer "F.Cu") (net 4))
 (segment (start 120.62 89.8) (end 120.62 90.8425) (width 0.8) (layer "F.Cu") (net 4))
 (segment (start 120.1 89.8) (end 120 89.9) (width 0.2) (layer "F.Cu") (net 4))
 (segment (start 123.625 91.238456) (end 123.625 90.5075) (width 0.2) (layer "F.Cu") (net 4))
 (segment (start 119.6 94.5375) (end 119.6 93) (width 0.8) (layer "F.Cu") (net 4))
 (segment (start 120.3625 95.3) (end 119.6 94.5375) (width 0.8) (layer "F.Cu") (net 4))
 (segment (start 120.3625 95.3) (end 120.3625 96) (width 0.8) (layer "F.Cu") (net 4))
 (segment (start 125.9 96.9) (end 125.78 96.78) (width 0.2) (layer "F.Cu") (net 4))
 (segment (start 120.62 90.8425) (end 120.4625 91) (width 0.8) (layer "F.Cu") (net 4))
 (segment (start 123.7 91.313456) (end 123.625 91.238456) (width 0.2) (layer "F.Cu") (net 4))
 (segment (start 119.8 93.5) (end 119.8 93.2) (width 0.2) (layer "F.Cu") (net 4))
 (segment (start 120.62 89.8) (end 120.1 89.8) (width 0.2) (layer "F.Cu") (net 4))
 (via (at 120.3625 95.3) (size 0.6) (drill 0.3) (layers "F.Cu" "B.Cu") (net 4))
 (via (at 123.7 91.7) (size 0.6) (drill 0.3) (layers "F.Cu" "B.Cu") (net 4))
 (via (at 119.6 93) (size 0.6) (drill 0.3) (layers "F.Cu" "B.Cu") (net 4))
 (via (at 119.9 90.5) (size 0.6) (drill 0.3) (layers "F.Cu" "B.Cu") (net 4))
 (via (at 125.9 96.9) (size 0.6) (drill 0.3) (layers "F.Cu" "B.Cu") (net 4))
 (via (at 120 89.9) (size 0.6) (drill 0.3) (layers "F.Cu" "B.Cu") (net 4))
 (segment (start 123.9 93.2) (end 123 92.3) (width 0.4) (layer "F.Cu") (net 7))
 (segment (start 121.675 95.7625) (end 121.9125 96) (width 0.2) (layer "F.Cu") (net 7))
 (segment (start 119.08 85.475) (end 119.08 91.333052) (width 0.2) (layer "F.Cu") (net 7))
 (segment (start 119.08 85.78) (end 119.08 85.475) (width 0.4) (layer "F.Cu") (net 7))
 (segment (start 124.3 93.2) (end 123.9 93.2) (width 0.4) (layer "F.Cu") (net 7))
 (segment (start 119.08 91.333052) (end 121.675 93.928052) (width 0.2) (layer "F.Cu") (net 7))
 (segment (start 124.925 93.825) (end 124.3 93.2) (width 0.4) (layer "F.Cu") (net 7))
 (segment (start 124.925 96.295) (end 124.82 96.4) (width 0.2) (layer "F.Cu") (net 7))
 (segment (start 123 89.7) (end 119.08 85.78) (width 0.4) (layer "F.Cu") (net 7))
 (segment (start 123 92.3) (end 123 89.7) (width 0.4) (layer "F.Cu") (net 7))
 (segment (start 124.82 96.48) (end 124.82 96.4) (width 0.2) (layer "F.Cu") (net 7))
 (segment (start 124.925 94.7325) (end 124.925 96.295) (width 0.2) (layer "F.Cu") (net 7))
 (segment (start 121.675 94.45) (end 121.675 95.7625) (width 0.2) (layer "F.Cu") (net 7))
 (segment (start 121.675 93.928052) (end 121.675 94.45) (width 0.2) (layer "F.Cu") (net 7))
 (segment (start 124.925 94.7325) (end 124.925 93.825) (width 0.4) (layer "F.Cu") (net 7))
 (segment (start 122.9 98.4) (end 124.82 96.48) (width 0.2) (layer "F.Cu") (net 7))
 (segment (start 124.38 88.8) (end 124.925 89.345) (width 0.2) (layer "F.Cu") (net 2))
 (segment (start 123.4 87.91) (end 123.49 87.91) (width 0.2) (layer "F.Cu") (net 2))
 (segment (start 124.925 89.345) (end 124.925 90.5075) (width 0.2) (layer "F.Cu") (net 2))
 (segment (start 123.49 87.91) (end 124.38 88.8) (width 0.2) (layer "F.Cu") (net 2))
 (segment (start 124.275 89.655) (end 124.275 90.5075) (width 0.2) (layer "F.Cu") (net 3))
 (segment (start 123.3 88.8) (end 123.42 88.8) (width 0.2) (layer "F.Cu") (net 3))
 (segment (start 123.42 88.8) (end 124.275 89.655) (width 0.2) (layer "F.Cu") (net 3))
 (segment (start 122.41 87.91) (end 123.3 88.8) (width 0.2) (layer "F.Cu") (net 3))
 (segment (start 122.4 87.91) (end 122.41 87.91) (width 0.2) (layer "F.Cu") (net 3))
 (segment (start 122.0125 92.2125) (end 122.0125 91) (width 0.5) (layer "F.Cu") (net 5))
 (segment (start 121.675 92.55) (end 121.675 92.775) (width 0.5) (layer "F.Cu") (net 5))
 (segment (start 122.0125 91) (end 122.0125 90.2325) (width 0.5) (layer "F.Cu") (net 5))
 (segment (start 121.675 92.775) (end 123.625 94.725) (width 0.5) (layer "F.Cu") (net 5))
 (segment (start 121.675 92.55) (end 122.0125 92.2125) (width 0.5) (layer "F.Cu") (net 5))
 (segment (start 122.0125 90.2325) (end 121.58 89.8) (width 0.5) (layer "F.Cu") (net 5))
 (segment (start 123.625 94.725) (end 123.625 94.7325) (width 0.5) (layer "F.Cu") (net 5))
 (segment (start 121.419999 98.4) (end 120.9 98.4) (width 0.2) (layer "F.Cu") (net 6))
 (segment (start 124.275 95.544999) (end 121.419999 98.4) (width 0.2) (layer "F.Cu") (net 6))
 (segment (start 124.275 94.7325) (end 124.275 95.544999) (width 0.2) (layer "F.Cu") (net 6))
 (segment (start 122.4 86.2) (end 122.4 86.89) (width 0.2) (layer "F.Cu") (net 9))
 (segment (start 121.62 85.475) (end 121.675 85.475) (width 0.2) (layer "F.Cu") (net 9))
 (segment (start 121.675 85.475) (end 122.4 86.2) (width 0.2) (layer "F.Cu") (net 9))
 (segment (start 123.4 86.89) (end 123.4 86.235) (width 0.2) (layer "F.Cu") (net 10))
 (segment (start 123.4 86.235) (end 124.16 85.475) (width 0.2) (layer "F.Cu") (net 10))
 (segment (start 126.9 93.4075) (end 125.575 94.7325) (width 0.2) (layer "F.Cu") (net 8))
 (segment (start 126.9 93.11) (end 126.9 93.4075) (width 0.2) (layer "F.Cu") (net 8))
 (segment (start 126.9 91.8325) (end 125.575 90.5075) (width 0.2) (layer "F.Cu") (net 1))
 (segment (start 126.9 92.09) (end 126.9 91.8325) (width 0.2) (layer "F.Cu") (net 1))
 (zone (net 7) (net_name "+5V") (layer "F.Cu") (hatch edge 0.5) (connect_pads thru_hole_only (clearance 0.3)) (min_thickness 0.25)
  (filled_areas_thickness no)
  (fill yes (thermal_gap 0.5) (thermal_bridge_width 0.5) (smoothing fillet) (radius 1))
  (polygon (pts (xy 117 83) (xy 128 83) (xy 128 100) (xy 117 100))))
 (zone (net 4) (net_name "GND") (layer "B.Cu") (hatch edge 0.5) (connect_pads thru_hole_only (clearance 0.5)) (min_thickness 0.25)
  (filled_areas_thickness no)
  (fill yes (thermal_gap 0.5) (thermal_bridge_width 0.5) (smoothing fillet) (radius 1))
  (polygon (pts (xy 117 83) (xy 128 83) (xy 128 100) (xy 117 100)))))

